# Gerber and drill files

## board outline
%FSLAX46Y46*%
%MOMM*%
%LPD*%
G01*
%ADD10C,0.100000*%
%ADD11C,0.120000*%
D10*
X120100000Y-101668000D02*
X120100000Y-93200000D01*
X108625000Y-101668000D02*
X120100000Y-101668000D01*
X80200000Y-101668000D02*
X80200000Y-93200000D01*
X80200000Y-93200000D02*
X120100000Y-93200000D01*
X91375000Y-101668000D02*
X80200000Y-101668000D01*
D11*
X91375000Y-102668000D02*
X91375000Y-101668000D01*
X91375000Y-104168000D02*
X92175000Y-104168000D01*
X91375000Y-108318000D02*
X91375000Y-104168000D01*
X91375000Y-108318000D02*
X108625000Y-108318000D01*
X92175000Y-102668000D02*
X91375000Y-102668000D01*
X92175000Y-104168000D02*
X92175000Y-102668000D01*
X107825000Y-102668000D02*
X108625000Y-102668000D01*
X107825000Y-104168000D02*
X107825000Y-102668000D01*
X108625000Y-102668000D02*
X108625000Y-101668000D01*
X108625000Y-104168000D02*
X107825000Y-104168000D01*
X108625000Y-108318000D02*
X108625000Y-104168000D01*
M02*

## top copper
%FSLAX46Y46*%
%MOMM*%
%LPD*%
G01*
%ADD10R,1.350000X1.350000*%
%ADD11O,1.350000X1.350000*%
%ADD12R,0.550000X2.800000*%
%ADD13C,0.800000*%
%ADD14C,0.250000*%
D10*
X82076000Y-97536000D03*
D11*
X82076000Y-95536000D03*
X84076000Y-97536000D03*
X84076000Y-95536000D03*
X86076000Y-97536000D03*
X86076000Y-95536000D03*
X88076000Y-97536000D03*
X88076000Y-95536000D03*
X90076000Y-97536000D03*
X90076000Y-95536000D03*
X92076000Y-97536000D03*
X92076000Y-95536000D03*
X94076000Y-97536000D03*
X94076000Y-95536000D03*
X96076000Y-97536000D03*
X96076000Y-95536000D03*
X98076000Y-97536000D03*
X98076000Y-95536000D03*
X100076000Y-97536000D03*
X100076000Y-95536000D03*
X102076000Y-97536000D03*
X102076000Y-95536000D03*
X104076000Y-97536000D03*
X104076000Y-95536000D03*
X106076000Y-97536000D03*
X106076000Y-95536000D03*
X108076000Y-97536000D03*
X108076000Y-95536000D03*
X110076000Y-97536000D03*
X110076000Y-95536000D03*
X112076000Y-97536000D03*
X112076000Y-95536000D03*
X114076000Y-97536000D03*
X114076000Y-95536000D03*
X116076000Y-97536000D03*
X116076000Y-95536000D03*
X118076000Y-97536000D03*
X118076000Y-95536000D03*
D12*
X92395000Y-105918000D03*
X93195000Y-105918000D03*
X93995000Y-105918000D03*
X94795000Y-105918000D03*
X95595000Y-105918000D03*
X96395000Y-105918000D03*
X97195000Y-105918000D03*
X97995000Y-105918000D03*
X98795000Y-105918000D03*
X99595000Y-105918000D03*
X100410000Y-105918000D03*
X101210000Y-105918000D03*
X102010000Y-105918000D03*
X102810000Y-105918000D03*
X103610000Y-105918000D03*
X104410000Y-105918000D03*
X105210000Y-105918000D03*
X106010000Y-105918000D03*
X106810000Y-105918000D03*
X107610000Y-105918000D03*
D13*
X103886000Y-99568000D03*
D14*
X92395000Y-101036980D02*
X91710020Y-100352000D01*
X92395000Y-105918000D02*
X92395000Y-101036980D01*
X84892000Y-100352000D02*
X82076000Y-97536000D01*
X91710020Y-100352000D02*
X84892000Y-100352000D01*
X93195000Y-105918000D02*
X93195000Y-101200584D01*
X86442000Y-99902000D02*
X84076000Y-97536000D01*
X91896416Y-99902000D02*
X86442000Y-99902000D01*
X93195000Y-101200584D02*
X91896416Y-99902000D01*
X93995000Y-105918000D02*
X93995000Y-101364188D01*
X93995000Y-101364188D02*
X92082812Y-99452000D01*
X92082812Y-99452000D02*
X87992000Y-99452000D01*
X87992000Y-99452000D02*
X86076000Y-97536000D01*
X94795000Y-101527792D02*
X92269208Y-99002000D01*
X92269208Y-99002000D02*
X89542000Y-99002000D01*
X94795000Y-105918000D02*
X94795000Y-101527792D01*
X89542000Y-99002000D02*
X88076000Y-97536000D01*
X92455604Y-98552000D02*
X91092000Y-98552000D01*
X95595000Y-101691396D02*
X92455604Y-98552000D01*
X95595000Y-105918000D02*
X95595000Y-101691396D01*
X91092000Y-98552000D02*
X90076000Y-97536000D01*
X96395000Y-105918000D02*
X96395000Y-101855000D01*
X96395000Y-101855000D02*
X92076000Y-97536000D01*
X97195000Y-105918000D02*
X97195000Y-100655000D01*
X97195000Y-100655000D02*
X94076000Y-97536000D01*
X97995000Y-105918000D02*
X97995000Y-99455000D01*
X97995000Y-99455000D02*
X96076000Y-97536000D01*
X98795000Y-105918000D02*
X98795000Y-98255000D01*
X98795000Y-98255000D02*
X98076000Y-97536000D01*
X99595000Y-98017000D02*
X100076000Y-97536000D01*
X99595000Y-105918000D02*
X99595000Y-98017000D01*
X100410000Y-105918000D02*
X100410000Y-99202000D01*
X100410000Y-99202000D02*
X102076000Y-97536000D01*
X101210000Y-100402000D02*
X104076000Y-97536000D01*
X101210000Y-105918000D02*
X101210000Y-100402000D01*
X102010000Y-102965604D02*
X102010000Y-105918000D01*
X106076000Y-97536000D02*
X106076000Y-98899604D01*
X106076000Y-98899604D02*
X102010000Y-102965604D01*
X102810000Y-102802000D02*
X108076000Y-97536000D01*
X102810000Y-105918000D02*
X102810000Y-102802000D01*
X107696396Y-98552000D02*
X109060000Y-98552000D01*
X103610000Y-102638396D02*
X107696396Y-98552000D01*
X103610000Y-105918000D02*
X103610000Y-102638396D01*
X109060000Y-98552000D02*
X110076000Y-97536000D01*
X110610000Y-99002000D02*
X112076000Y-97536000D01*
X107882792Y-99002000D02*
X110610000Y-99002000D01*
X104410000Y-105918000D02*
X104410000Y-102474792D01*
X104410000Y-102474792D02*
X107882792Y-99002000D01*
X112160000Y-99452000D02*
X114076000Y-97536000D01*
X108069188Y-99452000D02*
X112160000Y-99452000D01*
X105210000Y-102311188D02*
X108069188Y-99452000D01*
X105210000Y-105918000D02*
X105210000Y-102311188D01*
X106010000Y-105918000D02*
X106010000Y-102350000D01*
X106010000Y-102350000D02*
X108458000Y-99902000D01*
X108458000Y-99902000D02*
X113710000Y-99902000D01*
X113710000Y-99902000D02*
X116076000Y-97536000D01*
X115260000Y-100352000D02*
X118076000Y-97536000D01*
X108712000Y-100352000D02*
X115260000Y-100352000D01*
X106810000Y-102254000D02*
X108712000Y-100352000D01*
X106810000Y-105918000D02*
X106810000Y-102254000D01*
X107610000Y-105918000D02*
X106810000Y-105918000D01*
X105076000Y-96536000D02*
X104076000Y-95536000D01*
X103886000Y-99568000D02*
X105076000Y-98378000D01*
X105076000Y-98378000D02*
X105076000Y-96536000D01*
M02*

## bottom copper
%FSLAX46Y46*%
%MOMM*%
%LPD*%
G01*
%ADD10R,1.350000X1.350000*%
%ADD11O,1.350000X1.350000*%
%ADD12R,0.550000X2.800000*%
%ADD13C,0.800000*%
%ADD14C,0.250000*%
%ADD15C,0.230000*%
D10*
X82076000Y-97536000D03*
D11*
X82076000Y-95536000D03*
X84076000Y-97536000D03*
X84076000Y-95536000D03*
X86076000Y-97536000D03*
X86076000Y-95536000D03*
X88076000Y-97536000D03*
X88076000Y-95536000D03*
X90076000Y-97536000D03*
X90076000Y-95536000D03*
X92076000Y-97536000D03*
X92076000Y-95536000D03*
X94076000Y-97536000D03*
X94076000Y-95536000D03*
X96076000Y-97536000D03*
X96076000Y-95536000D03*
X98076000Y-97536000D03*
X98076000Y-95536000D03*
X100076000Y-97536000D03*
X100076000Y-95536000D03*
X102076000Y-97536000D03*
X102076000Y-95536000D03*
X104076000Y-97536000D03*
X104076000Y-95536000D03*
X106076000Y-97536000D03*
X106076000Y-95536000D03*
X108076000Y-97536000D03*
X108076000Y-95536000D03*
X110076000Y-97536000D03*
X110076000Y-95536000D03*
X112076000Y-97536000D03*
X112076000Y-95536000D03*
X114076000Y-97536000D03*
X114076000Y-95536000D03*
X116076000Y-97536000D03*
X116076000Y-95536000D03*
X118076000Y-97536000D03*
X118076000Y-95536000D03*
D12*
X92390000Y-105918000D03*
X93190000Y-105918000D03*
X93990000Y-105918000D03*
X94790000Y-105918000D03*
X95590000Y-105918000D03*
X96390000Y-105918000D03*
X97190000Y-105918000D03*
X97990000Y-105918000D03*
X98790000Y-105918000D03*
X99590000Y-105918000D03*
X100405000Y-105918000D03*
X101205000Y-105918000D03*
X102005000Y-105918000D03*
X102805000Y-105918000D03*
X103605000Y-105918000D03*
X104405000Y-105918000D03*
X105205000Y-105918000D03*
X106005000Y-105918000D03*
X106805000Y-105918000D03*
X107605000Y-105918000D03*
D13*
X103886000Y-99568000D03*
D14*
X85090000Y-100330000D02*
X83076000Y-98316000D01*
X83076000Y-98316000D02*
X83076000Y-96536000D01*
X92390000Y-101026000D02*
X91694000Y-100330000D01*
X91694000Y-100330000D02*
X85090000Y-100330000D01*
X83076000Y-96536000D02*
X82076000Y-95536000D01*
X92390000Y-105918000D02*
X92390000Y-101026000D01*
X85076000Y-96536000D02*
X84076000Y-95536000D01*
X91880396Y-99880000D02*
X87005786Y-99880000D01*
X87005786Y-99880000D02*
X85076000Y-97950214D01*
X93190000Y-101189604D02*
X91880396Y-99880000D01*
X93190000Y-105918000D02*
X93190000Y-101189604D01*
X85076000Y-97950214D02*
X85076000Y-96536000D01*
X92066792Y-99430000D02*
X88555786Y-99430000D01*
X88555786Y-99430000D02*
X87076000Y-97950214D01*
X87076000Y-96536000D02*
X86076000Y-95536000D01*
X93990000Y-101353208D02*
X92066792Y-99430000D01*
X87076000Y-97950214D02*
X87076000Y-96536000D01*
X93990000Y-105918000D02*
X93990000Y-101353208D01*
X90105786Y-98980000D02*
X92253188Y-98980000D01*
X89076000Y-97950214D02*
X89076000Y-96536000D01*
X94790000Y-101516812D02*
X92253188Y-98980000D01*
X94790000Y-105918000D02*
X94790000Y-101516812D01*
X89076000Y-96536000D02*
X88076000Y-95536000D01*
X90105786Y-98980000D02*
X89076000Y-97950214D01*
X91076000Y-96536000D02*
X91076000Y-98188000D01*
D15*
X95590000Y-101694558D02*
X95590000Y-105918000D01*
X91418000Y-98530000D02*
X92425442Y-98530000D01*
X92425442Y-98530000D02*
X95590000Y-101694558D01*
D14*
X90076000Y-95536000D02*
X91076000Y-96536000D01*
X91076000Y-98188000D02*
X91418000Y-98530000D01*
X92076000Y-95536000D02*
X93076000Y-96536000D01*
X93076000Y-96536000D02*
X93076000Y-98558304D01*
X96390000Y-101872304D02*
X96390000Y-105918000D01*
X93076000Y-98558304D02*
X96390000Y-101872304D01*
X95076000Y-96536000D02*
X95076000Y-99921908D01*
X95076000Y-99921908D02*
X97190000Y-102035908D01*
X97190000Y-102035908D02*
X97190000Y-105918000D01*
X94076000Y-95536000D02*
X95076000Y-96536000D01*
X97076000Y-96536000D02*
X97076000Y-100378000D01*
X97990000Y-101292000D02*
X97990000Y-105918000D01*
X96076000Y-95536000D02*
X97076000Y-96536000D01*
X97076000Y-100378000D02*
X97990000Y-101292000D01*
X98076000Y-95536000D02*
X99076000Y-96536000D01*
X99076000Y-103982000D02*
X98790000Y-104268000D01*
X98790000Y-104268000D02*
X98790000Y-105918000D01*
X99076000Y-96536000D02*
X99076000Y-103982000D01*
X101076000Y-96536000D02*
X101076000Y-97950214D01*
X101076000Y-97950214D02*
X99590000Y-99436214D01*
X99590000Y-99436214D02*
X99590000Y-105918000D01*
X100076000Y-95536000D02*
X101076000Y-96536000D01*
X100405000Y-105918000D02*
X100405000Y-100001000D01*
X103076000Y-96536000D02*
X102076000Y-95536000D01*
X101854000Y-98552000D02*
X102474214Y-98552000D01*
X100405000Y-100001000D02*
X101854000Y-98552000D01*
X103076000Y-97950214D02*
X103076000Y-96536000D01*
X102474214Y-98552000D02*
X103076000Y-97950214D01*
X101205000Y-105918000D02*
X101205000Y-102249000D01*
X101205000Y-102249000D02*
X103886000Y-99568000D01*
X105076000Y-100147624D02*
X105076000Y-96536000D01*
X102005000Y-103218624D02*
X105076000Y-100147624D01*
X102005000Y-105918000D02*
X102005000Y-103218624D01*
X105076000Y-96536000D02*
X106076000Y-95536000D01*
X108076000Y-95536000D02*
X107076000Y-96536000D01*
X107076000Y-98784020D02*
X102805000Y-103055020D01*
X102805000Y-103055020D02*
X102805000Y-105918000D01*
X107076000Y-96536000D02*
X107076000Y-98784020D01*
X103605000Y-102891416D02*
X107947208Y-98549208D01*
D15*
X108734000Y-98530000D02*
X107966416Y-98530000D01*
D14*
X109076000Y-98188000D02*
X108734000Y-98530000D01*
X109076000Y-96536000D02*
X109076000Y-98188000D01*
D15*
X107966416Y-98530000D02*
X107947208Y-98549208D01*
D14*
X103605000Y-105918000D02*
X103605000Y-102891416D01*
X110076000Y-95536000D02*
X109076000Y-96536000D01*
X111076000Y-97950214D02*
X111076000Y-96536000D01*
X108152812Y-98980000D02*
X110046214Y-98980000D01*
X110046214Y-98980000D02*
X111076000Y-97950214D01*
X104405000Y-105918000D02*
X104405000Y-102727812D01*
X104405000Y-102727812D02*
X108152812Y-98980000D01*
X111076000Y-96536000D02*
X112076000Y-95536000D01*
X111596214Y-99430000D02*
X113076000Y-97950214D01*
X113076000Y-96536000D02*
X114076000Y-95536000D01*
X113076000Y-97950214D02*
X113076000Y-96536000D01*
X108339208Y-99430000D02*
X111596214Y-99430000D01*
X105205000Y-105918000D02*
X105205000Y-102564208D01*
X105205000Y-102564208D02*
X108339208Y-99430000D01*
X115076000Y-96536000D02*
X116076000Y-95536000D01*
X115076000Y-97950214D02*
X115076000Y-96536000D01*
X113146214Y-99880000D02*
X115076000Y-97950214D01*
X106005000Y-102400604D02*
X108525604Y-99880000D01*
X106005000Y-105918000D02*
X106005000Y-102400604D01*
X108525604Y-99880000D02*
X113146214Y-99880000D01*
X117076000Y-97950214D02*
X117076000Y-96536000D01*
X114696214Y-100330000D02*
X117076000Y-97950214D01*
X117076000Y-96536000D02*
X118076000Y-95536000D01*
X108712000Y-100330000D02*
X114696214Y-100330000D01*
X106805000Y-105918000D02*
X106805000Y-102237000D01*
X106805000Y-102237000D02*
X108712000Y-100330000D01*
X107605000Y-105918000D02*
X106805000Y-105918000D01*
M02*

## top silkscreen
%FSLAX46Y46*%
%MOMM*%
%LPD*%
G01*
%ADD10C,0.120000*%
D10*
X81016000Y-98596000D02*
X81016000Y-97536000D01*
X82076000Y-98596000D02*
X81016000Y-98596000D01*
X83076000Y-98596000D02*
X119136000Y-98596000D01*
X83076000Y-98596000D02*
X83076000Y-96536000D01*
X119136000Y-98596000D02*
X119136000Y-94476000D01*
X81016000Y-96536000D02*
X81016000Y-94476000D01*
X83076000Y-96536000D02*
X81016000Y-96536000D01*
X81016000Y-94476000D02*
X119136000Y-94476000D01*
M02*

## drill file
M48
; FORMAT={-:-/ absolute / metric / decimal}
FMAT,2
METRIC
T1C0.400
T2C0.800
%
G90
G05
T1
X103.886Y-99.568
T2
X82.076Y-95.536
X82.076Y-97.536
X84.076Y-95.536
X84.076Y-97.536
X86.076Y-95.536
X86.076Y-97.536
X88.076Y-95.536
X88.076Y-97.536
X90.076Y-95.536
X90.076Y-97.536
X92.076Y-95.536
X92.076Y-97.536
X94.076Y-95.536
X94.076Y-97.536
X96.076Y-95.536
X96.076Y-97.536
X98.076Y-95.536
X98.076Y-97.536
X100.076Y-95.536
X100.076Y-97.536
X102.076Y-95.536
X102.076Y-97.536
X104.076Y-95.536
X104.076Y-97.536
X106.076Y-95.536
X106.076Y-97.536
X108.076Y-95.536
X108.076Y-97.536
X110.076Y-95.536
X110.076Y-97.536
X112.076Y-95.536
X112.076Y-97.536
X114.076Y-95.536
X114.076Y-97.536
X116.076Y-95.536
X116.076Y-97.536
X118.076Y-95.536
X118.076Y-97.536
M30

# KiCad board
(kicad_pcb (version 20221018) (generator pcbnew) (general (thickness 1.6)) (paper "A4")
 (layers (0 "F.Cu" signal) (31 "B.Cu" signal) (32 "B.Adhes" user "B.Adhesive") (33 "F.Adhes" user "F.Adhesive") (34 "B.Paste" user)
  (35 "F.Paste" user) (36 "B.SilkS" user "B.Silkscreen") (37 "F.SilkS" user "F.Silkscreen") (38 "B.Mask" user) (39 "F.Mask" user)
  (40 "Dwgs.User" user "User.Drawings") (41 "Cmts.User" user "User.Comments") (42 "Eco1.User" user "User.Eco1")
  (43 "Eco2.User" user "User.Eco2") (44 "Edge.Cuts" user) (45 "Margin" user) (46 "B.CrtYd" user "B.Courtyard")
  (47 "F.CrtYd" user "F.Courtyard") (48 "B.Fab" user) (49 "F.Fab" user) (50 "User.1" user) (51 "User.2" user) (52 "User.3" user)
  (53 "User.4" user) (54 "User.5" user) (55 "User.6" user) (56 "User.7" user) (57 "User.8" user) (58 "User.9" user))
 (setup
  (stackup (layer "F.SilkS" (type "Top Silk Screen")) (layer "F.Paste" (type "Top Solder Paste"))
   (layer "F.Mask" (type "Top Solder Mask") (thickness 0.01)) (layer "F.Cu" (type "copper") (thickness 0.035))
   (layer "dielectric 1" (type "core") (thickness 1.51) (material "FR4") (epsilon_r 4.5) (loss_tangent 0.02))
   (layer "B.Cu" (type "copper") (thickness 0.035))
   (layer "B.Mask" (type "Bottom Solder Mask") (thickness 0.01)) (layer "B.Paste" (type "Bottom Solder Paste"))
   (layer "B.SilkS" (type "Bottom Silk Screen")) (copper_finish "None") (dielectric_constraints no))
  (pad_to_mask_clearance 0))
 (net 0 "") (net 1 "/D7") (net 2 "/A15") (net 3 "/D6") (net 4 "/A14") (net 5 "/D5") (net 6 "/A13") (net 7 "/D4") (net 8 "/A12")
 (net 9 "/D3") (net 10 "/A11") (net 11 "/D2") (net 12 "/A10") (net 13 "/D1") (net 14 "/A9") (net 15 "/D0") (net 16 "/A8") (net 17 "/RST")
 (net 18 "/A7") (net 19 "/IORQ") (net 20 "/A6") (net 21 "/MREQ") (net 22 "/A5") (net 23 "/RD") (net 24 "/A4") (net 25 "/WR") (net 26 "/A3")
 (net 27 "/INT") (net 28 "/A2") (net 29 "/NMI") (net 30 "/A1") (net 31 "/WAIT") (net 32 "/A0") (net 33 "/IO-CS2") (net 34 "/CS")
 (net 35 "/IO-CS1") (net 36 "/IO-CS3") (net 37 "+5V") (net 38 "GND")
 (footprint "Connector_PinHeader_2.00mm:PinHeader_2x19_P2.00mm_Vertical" (layer "F.Cu") (at 82.076 97.536 90)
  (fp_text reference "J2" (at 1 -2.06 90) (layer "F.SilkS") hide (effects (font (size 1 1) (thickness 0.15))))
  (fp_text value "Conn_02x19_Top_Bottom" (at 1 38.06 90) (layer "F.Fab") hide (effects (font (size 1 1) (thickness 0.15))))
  (fp_line (start -1.06 -1.06) (end 0 -1.06) (stroke (width 0.12) (type solid)) (layer "F.SilkS"))
  (fp_line (start -1.06 0) (end -1.06 -1.06) (stroke (width 0.12) (type solid)) (layer "F.SilkS"))
  (fp_line (start -1.06 1) (end -1.06 37.06) (stroke (width 0.12) (type solid)) (layer "F.SilkS"))
  (fp_line (start -1.06 1) (end 1 1) (stroke (width 0.12) (type solid)) (layer "F.SilkS"))
  (fp_line (start -1.06 37.06) (end 3.06 37.06) (stroke (width 0.12) (type solid)) (layer "F.SilkS"))
  (fp_line (start 1 -1.06) (end 3.06 -1.06) (stroke (width 0.12) (type solid)) (layer "F.SilkS"))
  (fp_line (start 1 1) (end 1 -1.06) (stroke (width 0.12) (type solid)) (layer "F.SilkS"))
  (fp_line (start 3.06 -1.06) (end 3.06 37.06) (stroke (width 0.12) (type solid)) (layer "F.SilkS"))
  (pad "1" thru_hole rect (at 0 0 90) (size 1.35 1.35) (drill 0.8) (layers "*.Cu" "*.Mask") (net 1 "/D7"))
  (pad "2" thru_hole oval (at 2 0 90) (size 1.35 1.35) (drill 0.8) (layers "*.Cu" "*.Mask") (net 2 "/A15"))
  (pad "3" thru_hole oval (at 0 2 90) (size 1.35 1.35) (drill 0.8) (layers "*.Cu" "*.Mask") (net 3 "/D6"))
  (pad "4" thru_hole oval (at 2 2 90) (size 1.35 1.35) (drill 0.8) (layers "*.Cu" "*.Mask") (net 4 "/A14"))
  (pad "5" thru_hole oval (at 0 4 90) (size 1.35 1.35) (drill 0.8) (layers "*.Cu" "*.Mask") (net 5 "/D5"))
  (pad "6" thru_hole oval (at 2 4 90) (size 1.35 1.35) (drill 0.8) (layers "*.Cu" "*.Mask") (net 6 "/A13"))
  (pad "7" thru_hole oval (at 0 6 90) (size 1.35 1.35) (drill 0.8) (layers "*.Cu" "*.Mask") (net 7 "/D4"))
  (pad "8" thru_hole oval (at 2 6 90) (size 1.35 1.35) (drill 0.8) (layers "*.Cu" "*.Mask") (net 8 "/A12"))
  (pad "9" thru_hole oval (at 0 8 90) (size 1.35 1.35) (drill 0.8) (layers "*.Cu" "*.Mask") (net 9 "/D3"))
  (pad "10" thru_hole oval (at 2 8 90) (size 1.35 1.35) (drill 0.8) (layers "*.Cu" "*.Mask") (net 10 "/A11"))
  (pad "11" thru_hole oval (at 0 10 90) (size 1.35 1.35) (drill 0.8) (layers "*.Cu" "*.Mask") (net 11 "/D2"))
  (pad "12" thru_hole oval (at 2 10 90) (size 1.35 1.35) (drill 0.8) (layers "*.Cu" "*.Mask") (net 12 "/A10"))
  (pad "13" thru_hole oval (at 0 12 90) (size 1.35 1.35) (drill 0.8) (layers "*.Cu" "*.Mask") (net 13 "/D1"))
  (pad "14" thru_hole oval (at 2 12 90) (size 1.35 1.35) (drill 0.8) (layers "*.Cu" "*.Mask") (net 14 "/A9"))
  (pad "15" thru_hole oval (at 0 14 90) (size 1.35 1.35) (drill 0.8) (layers "*.Cu" "*.Mask") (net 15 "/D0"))
  (pad "16" thru_hole oval (at 2 14 90) (size 1.35 1.35) (drill 0.8) (layers "*.Cu" "*.Mask") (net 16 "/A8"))
  (pad "17" thru_hole oval (at 0 16 90) (size 1.35 1.35) (drill 0.8) (layers "*.Cu" "*.Mask") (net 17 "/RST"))
  (pad "18" thru_hole oval (at 2 16 90) (size 1.35 1.35) (drill 0.8) (layers "*.Cu" "*.Mask") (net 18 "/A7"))
  (pad "19" thru_hole oval (at 0 18 90) (size 1.35 1.35) (drill 0.8) (layers "*.Cu" "*.Mask") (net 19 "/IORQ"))
  (pad "20" thru_hole oval (at 2 18 90) (size 1.35 1.35) (drill 0.8) (layers "*.Cu" "*.Mask") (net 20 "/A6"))
  (pad "21" thru_hole oval (at 0 20 90) (size 1.35 1.35) (drill 0.8) (layers "*.Cu" "*.Mask") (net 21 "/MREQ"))
  (pad "22" thru_hole oval (at 2 20 90) (size 1.35 1.35) (drill 0.8) (layers "*.Cu" "*.Mask") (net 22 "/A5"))
  (pad "23" thru_hole oval (at 0 22 90) (size 1.35 1.35) (drill 0.8) (layers "*.Cu" "*.Mask") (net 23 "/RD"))
  (pad "24" thru_hole oval (at 2 22 90) (size 1.35 1.35) (drill 0.8) (layers "*.Cu" "*.Mask") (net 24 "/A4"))
  (pad "25" thru_hole oval (at 0 24 90) (size 1.35 1.35) (drill 0.8) (layers "*.Cu" "*.Mask") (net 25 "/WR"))
  (pad "26" thru_hole oval (at 2 24 90) (size 1.35 1.35) (drill 0.8) (layers "*.Cu" "*.Mask") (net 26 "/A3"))
  (pad "27" thru_hole oval (at 0 26 90) (size 1.35 1.35) (drill 0.8) (layers "*.Cu" "*.Mask") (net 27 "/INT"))
  (pad "28" thru_hole oval (at 2 26 90) (size 1.35 1.35) (drill 0.8) (layers "*.Cu" "*.Mask") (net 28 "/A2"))
  (pad "29" thru_hole oval (at 0 28 90) (size 1.35 1.35) (drill 0.8) (layers "*.Cu" "*.Mask") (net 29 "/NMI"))
  (pad "30" thru_hole oval (at 2 28 90) (size 1.35 1.35) (drill 0.8) (layers "*.Cu" "*.Mask") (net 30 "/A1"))
  (pad "31" thru_hole oval (at 0 30 90) (size 1.35 1.35) (drill 0.8) (layers "*.Cu" "*.Mask") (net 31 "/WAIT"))
  (pad "32" thru_hole oval (at 2 30 90) (size 1.35 1.35) (drill 0.8) (layers "*.Cu" "*.Mask") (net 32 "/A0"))
  (pad "33" thru_hole oval (at 0 32 90) (size 1.35 1.35) (drill 0.8) (layers "*.Cu" "*.Mask") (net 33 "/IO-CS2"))
  (pad "34" thru_hole oval (at 2 32 90) (size 1.35 1.35) (drill 0.8) (layers "*.Cu" "*.Mask") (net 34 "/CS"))
  (pad "35" thru_hole oval (at 0 34 90) (size 1.35 1.35) (drill 0.8) (layers "*.Cu" "*.Mask") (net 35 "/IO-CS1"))
  (pad "36" thru_hole oval (at 2 34 90) (size 1.35 1.35) (drill 0.8) (layers "*.Cu" "*.Mask") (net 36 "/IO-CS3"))
  (pad "37" thru_hole oval (at 0 36 90) (size 1.35 1.35) (drill 0.8) (layers "*.Cu" "*.Mask") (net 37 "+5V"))
  (pad "38" thru_hole oval (at 2 36 90) (size 1.35 1.35) (drill 0.8) (layers "*.Cu" "*.Mask") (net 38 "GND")))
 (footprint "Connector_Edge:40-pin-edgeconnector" (layer "F.Cu") (at 100 103.378)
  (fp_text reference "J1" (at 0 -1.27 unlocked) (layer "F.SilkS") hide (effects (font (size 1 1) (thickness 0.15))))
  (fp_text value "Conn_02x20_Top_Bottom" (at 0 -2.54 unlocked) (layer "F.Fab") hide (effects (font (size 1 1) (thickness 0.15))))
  (fp_line (start -8.625 -0.71) (end -8.625 -1.71) (stroke (width 0.12) (type default)) (layer "Edge.Cuts"))
  (fp_line (start -8.625 0.79) (end -7.825 0.79) (stroke (width 0.12) (type default)) (layer "Edge.Cuts"))
  (fp_line (start -8.625 4.94) (end -8.625 0.79) (stroke (width 0.12) (type default)) (layer "Edge.Cuts"))
  (fp_line (start -8.625 4.94) (end 8.625 4.94) (stroke (width 0.12) (type default)) (layer "Edge.Cuts"))
  (fp_line (start -7.825 -0.71) (end -8.625 -0.71) (stroke (width 0.12) (type default)) (layer "Edge.Cuts"))
  (fp_line (start -7.825 0.79) (end -7.825 -0.71) (stroke (width 0.12) (type default)) (layer "Edge.Cuts"))
  (fp_line (start 7.825 -0.71) (end 8.625 -0.71) (stroke (width 0.12) (type default)) (layer "Edge.Cuts"))
  (fp_line (start 7.825 0.79) (end 7.825 -0.71) (stroke (width 0.12) (type default)) (layer "Edge.Cuts"))
  (fp_line (start 8.625 -0.71) (end 8.625 -1.71) (stroke (width 0.12) (type default)) (layer "Edge.Cuts"))
  (fp_line (start 8.625 0.79) (end 7.825 0.79) (stroke (width 0.12) (type default)) (layer "Edge.Cuts"))
  (fp_line (start 8.625 4.94) (end 8.625 0.79) (stroke (width 0.12) (type default)) (layer "Edge.Cuts"))
  (pad "1" smd rect (at -7.605 2.54 90) (size 2.8 0.55) (layers "F.Cu" "F.Paste" "F.Mask") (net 1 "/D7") (thermal_bridge_angle 45))
  (pad "2" smd rect (at -6.805 2.54 90) (size 2.8 0.55) (layers "F.Cu" "F.Paste" "F.Mask") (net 3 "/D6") (thermal_bridge_angle 45))
  (pad "3" smd rect (at -6.005 2.54 90) (size 2.8 0.55) (layers "F.Cu" "F.Paste" "F.Mask") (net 5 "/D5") (thermal_bridge_angle 45))
  (pad "4" smd rect (at -5.205 2.54 90) (size 2.8 0.55) (layers "F.Cu" "F.Paste" "F.Mask") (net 7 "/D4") (thermal_bridge_angle 45))
  (pad "5" smd rect (at -4.405 2.54 90) (size 2.8 0.55) (layers "F.Cu" "F.Paste" "F.Mask") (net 9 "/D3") (thermal_bridge_angle 45))
  (pad "6" smd rect (at -3.605 2.54 90) (size 2.8 0.55) (layers "F.Cu" "F.Paste" "F.Mask") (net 11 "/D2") (thermal_bridge_angle 45))
  (pad "7" smd rect (at -2.805 2.54 90) (size 2.8 0.55) (layers "F.Cu" "F.Paste" "F.Mask") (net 13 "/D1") (thermal_bridge_angle 45))
  (pad "8" smd rect (at -2.005 2.54 90) (size 2.8 0.55) (layers "F.Cu" "F.Paste" "F.Mask") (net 15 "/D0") (thermal_bridge_angle 45))
  (pad "9" smd rect (at -1.205 2.54 90) (size 2.8 0.55) (layers "F.Cu" "F.Paste" "F.Mask") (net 17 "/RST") (thermal_bridge_angle 45))
  (pad "10" smd rect (at -0.405 2.54 90) (size 2.8 0.55) (layers "F.Cu" "F.Paste" "F.Mask") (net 19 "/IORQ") (thermal_bridge_angle 45))
  (pad "11" smd rect (at 0.41 2.54 90) (size 2.8 0.55) (layers "F.Cu" "F.Paste" "F.Mask") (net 21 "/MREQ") (thermal_bridge_angle 45))
  (pad "12" smd rect (at 1.21 2.54 90) (size 2.8 0.55) (layers "F.Cu" "F.Paste" "F.Mask") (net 23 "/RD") (thermal_bridge_angle 45))
  (pad "13" smd rect (at 2.01 2.54 90) (size 2.8 0.55) (layers "F.Cu" "F.Paste" "F.Mask") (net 25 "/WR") (thermal_bridge_angle 45))
  (pad "14" smd rect (at 2.81 2.54 90) (size 2.8 0.55) (layers "F.Cu" "F.Paste" "F.Mask") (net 27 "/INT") (thermal_bridge_angle 45))
  (pad "15" smd rect (at 3.61 2.54 90) (size 2.8 0.55) (layers "F.Cu" "F.Paste" "F.Mask") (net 29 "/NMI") (thermal_bridge_angle 45))
  (pad "16" smd rect (at 4.41 2.54 90) (size 2.8 0.55) (layers "F.Cu" "F.Paste" "F.Mask") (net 31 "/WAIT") (thermal_bridge_angle 45))
  (pad "17" smd rect (at 5.21 2.54 90) (size 2.8 0.55) (layers "F.Cu" "F.Paste" "F.Mask") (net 33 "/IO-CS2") (thermal_bridge_angle 45))
  (pad "18" smd rect (at 6.01 2.54 90) (size 2.8 0.55) (layers "F.Cu" "F.Paste" "F.Mask") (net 35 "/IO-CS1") (thermal_bridge_angle 45))
  (pad "19" smd rect (at 6.81 2.54 90) (size 2.8 0.55) (layers "F.Cu" "F.Paste" "F.Mask") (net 37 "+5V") (thermal_bridge_angle 45))
  (pad "20" smd rect (at 7.61 2.54 90) (size 2.8 0.55) (layers "F.Cu" "F.Paste" "F.Mask") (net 37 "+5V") (thermal_bridge_angle 45))
  (pad "21" smd rect (at -7.61 2.54 270) (size 2.8 0.55) (layers "B.Cu" "B.Paste" "B.Mask") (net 2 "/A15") (thermal_bridge_angle 45))
  (pad "22" smd rect (at -6.81 2.54 270) (size 2.8 0.55) (layers "B.Cu" "B.Paste" "B.Mask") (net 4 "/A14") (thermal_bridge_angle 45))
  (pad "23" smd rect (at -6.01 2.54 270) (size 2.8 0.55) (layers "B.Cu" "B.Paste" "B.Mask") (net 6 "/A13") (thermal_bridge_angle 45))
  (pad "24" smd rect (at -5.21 2.54 270) (size 2.8 0.55) (layers "B.Cu" "B.Paste" "B.Mask") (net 8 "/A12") (thermal_bridge_angle 45))
  (pad "25" smd rect (at -4.41 2.54 270) (size 2.8 0.55) (layers "B.Cu" "B.Paste" "B.Mask") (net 10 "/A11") (thermal_bridge_angle 45))
  (pad "26" smd rect (at -3.61 2.54 270) (size 2.8 0.55) (layers "B.Cu" "B.Paste" "B.Mask") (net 12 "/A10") (thermal_bridge_angle 45))
  (pad "27" smd rect (at -2.81 2.54 270) (size 2.8 0.55) (layers "B.Cu" "B.Paste" "B.Mask") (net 14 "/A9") (thermal_bridge_angle 45))
  (pad "28" smd rect (at -2.01 2.54 270) (size 2.8 0.55) (layers "B.Cu" "B.Paste" "B.Mask") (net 16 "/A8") (thermal_bridge_angle 45))
  (pad "29" smd rect (at -1.21 2.54 270) (size 2.8 0.55) (layers "B.Cu" "B.Paste" "B.Mask") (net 18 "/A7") (thermal_bridge_angle 45))
  (pad "30" smd rect (at -0.41 2.54 270) (size 2.8 0.55) (layers "B.Cu" "B.Paste" "B.Mask") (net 20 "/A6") (thermal_bridge_angle 45))
  (pad "31" smd rect (at 0.405 2.54 270) (size 2.8 0.55) (layers "B.Cu" "B.Paste" "B.Mask") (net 22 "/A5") (thermal_bridge_angle 45))
  (pad "32" smd rect (at 1.205 2.54 270) (size 2.8 0.55) (layers "B.Cu" "B.Paste" "B.Mask") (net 24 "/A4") (thermal_bridge_angle 45))
  (pad "33" smd rect (at 2.005 2.54 270) (size 2.8 0.55) (layers "B.Cu" "B.Paste" "B.Mask") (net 26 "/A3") (thermal_bridge_angle 45))
  (pad "34" smd rect (at 2.805 2.54 270) (size 2.8 0.55) (layers "B.Cu" "B.Paste" "B.Mask") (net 28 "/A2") (thermal_bridge_angle 45))
  (pad "35" smd rect (at 3.605 2.54 270) (size 2.8 0.55) (layers "B.Cu" "B.Paste" "B.Mask") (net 30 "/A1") (thermal_bridge_angle 45))
  (pad "36" smd rect (at 4.405 2.54 270) (size 2.8 0.55) (layers "B.Cu" "B.Paste" "B.Mask") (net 32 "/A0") (thermal_bridge_angle 45))
  (pad "37" smd rect (at 5.205 2.54 270) (size 2.8 0.55) (layers "B.Cu" "B.Paste" "B.Mask") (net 34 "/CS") (thermal_bridge_angle 45))
  (pad "38" smd rect (at 6.005 2.54 270) (size 2.8 0.55) (layers "B.Cu" "B.Paste" "B.Mask") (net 36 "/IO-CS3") (thermal_bridge_angle 45))
  (pad "39" smd rect (at 6.805 2.54 270) (size 2.8 0.55) (layers "B.Cu" "B.Paste" "B.Mask") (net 38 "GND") (thermal_bridge_angle 45))
  (pad "40" smd rect (at 7.605 2.54 270) (size 2.8 0.55) (layers "B.Cu" "B.Paste" "B.Mask") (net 38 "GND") (thermal_bridge_angle 45)))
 (gr_line (start 120.1 101.668) (end 120.1 93.2) (stroke (width 0.1) (type default)) (layer "Edge.Cuts"))
 (gr_line (start 108.625 101.668) (end 120.1 101.668) (stroke (width 0.1) (type default)) (layer "Edge.Cuts"))
 (gr_line (start 80.2 101.668) (end 80.2 93.2) (stroke (width 0.1) (type default)) (layer "Edge.Cuts"))
 (gr_line (start 80.2 93.2) (end 120.1 93.2) (stroke (width 0.1) (type default)) (layer "Edge.Cuts"))
 (gr_line (start 91.375 101.668) (end 80.2 101.668) (stroke (width 0.1) (type default)) (layer "Edge.Cuts"))
 (segment (start 92.395 101.03698) (end 91.71002 100.352) (width 0.25) (layer "F.Cu") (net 1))
 (segment (start 92.395 105.918) (end 92.395 101.03698) (width 0.25) (layer "F.Cu") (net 1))
 (segment (start 84.892 100.352) (end 82.076 97.536) (width 0.25) (layer "F.Cu") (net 1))
 (segment (start 91.71002 100.352) (end 84.892 100.352) (width 0.25) (layer "F.Cu") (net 1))
 (segment (start 93.195 105.918) (end 93.195 101.200584) (width 0.25) (layer "F.Cu") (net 3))
 (segment (start 86.442 99.902) (end 84.076 97.536) (width 0.25) (layer "F.Cu") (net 3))
 (segment (start 91.896416 99.902) (end 86.442 99.902) (width 0.25) (layer "F.Cu") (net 3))
 (segment (start 93.195 101.200584) (end 91.896416 99.902) (width 0.25) (layer "F.Cu") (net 3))
 (segment (start 93.995 105.918) (end 93.995 101.364188) (width 0.25) (layer "F.Cu") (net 5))
 (segment (start 93.995 101.364188) (end 92.082812 99.452) (width 0.25) (layer "F.Cu") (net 5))
 (segment (start 92.082812 99.452) (end 87.992 99.452) (width 0.25) (layer "F.Cu") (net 5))
 (segment (start 87.992 99.452) (end 86.076 97.536) (width 0.25) (layer "F.Cu") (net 5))
 (segment (start 94.795 101.527792) (end 92.269208 99.002) (width 0.25) (layer "F.Cu") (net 7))
 (segment (start 92.269208 99.002) (end 89.542 99.002) (width 0.25) (layer "F.Cu") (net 7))
 (segment (start 94.795 105.918) (end 94.795 101.527792) (width 0.25) (layer "F.Cu") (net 7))
 (segment (start 89.542 99.002) (end 88.076 97.536) (width 0.25) (layer "F.Cu") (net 7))
 (segment (start 92.455604 98.552) (end 91.092 98.552) (width 0.25) (layer "F.Cu") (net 9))
 (segment (start 95.595 101.691396) (end 92.455604 98.552) (width 0.25) (layer "F.Cu") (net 9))
 (segment (start 95.595 105.918) (end 95.595 101.691396) (width 0.25) (layer "F.Cu") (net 9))
 (segment (start 91.092 98.552) (end 90.076 97.536) (width 0.25) (layer "F.Cu") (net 9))
 (segment (start 96.395 105.918) (end 96.395 101.855) (width 0.25) (layer "F.Cu") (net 11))
 (segment (start 96.395 101.855) (end 92.076 97.536) (width 0.25) (layer "F.Cu") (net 11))
 (segment (start 97.195 105.918) (end 97.195 100.655) (width 0.25) (layer "F.Cu") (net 13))
 (segment (start 97.195 100.655) (end 94.076 97.536) (width 0.25) (layer "F.Cu") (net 13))
 (segment (start 97.995 105.918) (end 97.995 99.455) (width 0.25) (layer "F.Cu") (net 15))
 (segment (start 97.995 99.455) (end 96.076 97.536) (width 0.25) (layer "F.Cu") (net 15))
 (segment (start 98.795 105.918) (end 98.795 98.255) (width 0.25) (layer "F.Cu") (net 17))
 (segment (start 98.795 98.255) (end 98.076 97.536) (width 0.25) (layer "F.Cu") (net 17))
 (segment (start 99.595 98.017) (end 100.076 97.536) (width 0.25) (layer "F.Cu") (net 19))
 (segment (start 99.595 105.918) (end 99.595 98.017) (width 0.25) (layer "F.Cu") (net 19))
 (segment (start 100.41 105.918) (end 100.41 99.202) (width 0.25) (layer "F.Cu") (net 21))
 (segment (start 100.41 99.202) (end 102.076 97.536) (width 0.25) (layer "F.Cu") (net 21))
 (segment (start 101.21 100.402) (end 104.076 97.536) (width 0.25) (layer "F.Cu") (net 23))
 (segment (start 101.21 105.918) (end 101.21 100.402) (width 0.25) (layer "F.Cu") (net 23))
 (segment (start 102.01 102.965604) (end 102.01 105.918) (width 0.25) (layer "F.Cu") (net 25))
 (segment (start 106.076 97.536) (end 106.076 98.899604) (width 0.25) (layer "F.Cu") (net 25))
 (segment (start 106.076 98.899604) (end 102.01 102.965604) (width 0.25) (layer "F.Cu") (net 25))
 (segment (start 102.81 102.802) (end 108.076 97.536) (width 0.25) (layer "F.Cu") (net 27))
 (segment (start 102.81 105.918) (end 102.81 102.802) (width 0.25) (layer "F.Cu") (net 27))
 (segment (start 107.696396 98.552) (end 109.06 98.552) (width 0.25) (layer "F.Cu") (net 29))
 (segment (start 103.61 102.638396) (end 107.696396 98.552) (width 0.25) (layer "F.Cu") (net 29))
 (segment (start 103.61 105.918) (end 103.61 102.638396) (width 0.25) (layer "F.Cu") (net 29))
 (segment (start 109.06 98.552) (end 110.076 97.536) (width 0.25) (layer "F.Cu") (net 29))
 (segment (start 110.61 99.002) (end 112.076 97.536) (width 0.25) (layer "F.Cu") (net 31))
 (segment (start 107.882792 99.002) (end 110.61 99.002) (width 0.25) (layer "F.Cu") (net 31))
 (segment (start 104.41 105.918) (end 104.41 102.474792) (width 0.25) (layer "F.Cu") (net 31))
 (segment (start 104.41 102.474792) (end 107.882792 99.002) (width 0.25) (layer "F.Cu") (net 31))
 (segment (start 112.16 99.452) (end 114.076 97.536) (width 0.25) (layer "F.Cu") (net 33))
 (segment (start 108.069188 99.452) (end 112.16 99.452) (width 0.25) (layer "F.Cu") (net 33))
 (segment (start 105.21 102.311188) (end 108.069188 99.452) (width 0.25) (layer "F.Cu") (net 33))
 (segment (start 105.21 105.918) (end 105.21 102.311188) (width 0.25) (layer "F.Cu") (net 33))
 (segment (start 106.01 105.918) (end 106.01 102.35) (width 0.25) (layer "F.Cu") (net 35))
 (segment (start 106.01 102.35) (end 108.458 99.902) (width 0.25) (layer "F.Cu") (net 35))
 (segment (start 108.458 99.902) (end 113.71 99.902) (width 0.25) (layer "F.Cu") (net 35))
 (segment (start 113.71 99.902) (end 116.076 97.536) (width 0.25) (layer "F.Cu") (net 35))
 (segment (start 115.26 100.352) (end 118.076 97.536) (width 0.25) (layer "F.Cu") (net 37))
 (segment (start 108.712 100.352) (end 115.26 100.352) (width 0.25) (layer "F.Cu") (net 37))
 (segment (start 106.81 102.254) (end 108.712 100.352) (width 0.25) (layer "F.Cu") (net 37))
 (segment (start 106.81 105.918) (end 106.81 102.254) (width 0.25) (layer "F.Cu") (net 37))
 (segment (start 107.61 105.918) (end 106.81 105.918) (width 0.25) (layer "F.Cu") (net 37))
 (segment (start 85.09 100.33) (end 83.076 98.316) (width 0.25) (layer "B.Cu") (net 2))
 (segment (start 83.076 98.316) (end 83.076 96.536) (width 0.25) (layer "B.Cu") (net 2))
 (segment (start 92.39 101.026) (end 91.694 100.33) (width 0.25) (layer "B.Cu") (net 2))
 (segment (start 91.694 100.33) (end 85.09 100.33) (width 0.25) (layer "B.Cu") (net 2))
 (segment (start 83.076 96.536) (end 82.076 95.536) (width 0.25) (layer "B.Cu") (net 2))
 (segment (start 92.39 105.918) (end 92.39 101.026) (width 0.25) (layer "B.Cu") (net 2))
 (segment (start 85.076 96.536) (end 84.076 95.536) (width 0.25) (layer "B.Cu") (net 4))
 (segment (start 91.880396 99.88) (end 87.005786 99.88) (width 0.25) (layer "B.Cu") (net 4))
 (segment (start 87.005786 99.88) (end 85.076 97.950214) (width 0.25) (layer "B.Cu") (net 4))
 (segment (start 93.19 101.189604) (end 91.880396 99.88) (width 0.25) (layer "B.Cu") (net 4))
 (segment (start 93.19 105.918) (end 93.19 101.189604) (width 0.25) (layer "B.Cu") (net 4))
 (segment (start 85.076 97.950214) (end 85.076 96.536) (width 0.25) (layer "B.Cu") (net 4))
 (segment (start 92.066792 99.43) (end 88.555786 99.43) (width 0.25) (layer "B.Cu") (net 6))
 (segment (start 88.555786 99.43) (end 87.076 97.950214) (width 0.25) (layer "B.Cu") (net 6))
 (segment (start 87.076 96.536) (end 86.076 95.536) (width 0.25) (layer "B.Cu") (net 6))
 (segment (start 93.99 101.353208) (end 92.066792 99.43) (width 0.25) (layer "B.Cu") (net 6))
 (segment (start 87.076 97.950214) (end 87.076 96.536) (width 0.25) (layer "B.Cu") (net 6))
 (segment (start 93.99 105.918) (end 93.99 101.353208) (width 0.25) (layer "B.Cu") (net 6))
 (segment (start 90.105786 98.98) (end 92.253188 98.98) (width 0.25) (layer "B.Cu") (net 8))
 (segment (start 89.076 97.950214) (end 89.076 96.536) (width 0.25) (layer "B.Cu") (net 8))
 (segment (start 94.79 101.516812) (end 92.253188 98.98) (width 0.25) (layer "B.Cu") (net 8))
 (segment (start 94.79 105.918) (end 94.79 101.516812) (width 0.25) (layer "B.Cu") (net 8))
 (segment (start 89.076 96.536) (end 88.076 95.536) (width 0.25) (layer "B.Cu") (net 8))
 (segment (start 90.105786 98.98) (end 89.076 97.950214) (width 0.25) (layer "B.Cu") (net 8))
 (segment (start 91.076 96.536) (end 91.076 98.188) (width 0.25) (layer "B.Cu") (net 10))
 (segment (start 95.59 101.694558) (end 95.59 105.918) (width 0.23) (layer "B.Cu") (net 10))
 (segment (start 91.418 98.53) (end 92.425442 98.53) (width 0.23) (layer "B.Cu") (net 10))
 (segment (start 92.425442 98.53) (end 95.59 101.694558) (width 0.23) (layer "B.Cu") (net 10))
 (segment (start 90.076 95.536) (end 91.076 96.536) (width 0.25) (layer "B.Cu") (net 10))
 (segment (start 91.076 98.188) (end 91.418 98.53) (width 0.25) (layer "B.Cu") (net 10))
 (segment (start 92.076 95.536) (end 93.076 96.536) (width 0.25) (layer "B.Cu") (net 12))
 (segment (start 93.076 96.536) (end 93.076 98.558304) (width 0.25) (layer "B.Cu") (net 12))
 (segment (start 96.39 101.872304) (end 96.39 105.918) (width 0.25) (layer "B.Cu") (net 12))
 (segment (start 93.076 98.558304) (end 96.39 101.872304) (width 0.25) (layer "B.Cu") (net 12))
 (segment (start 95.076 96.536) (end 95.076 99.921908) (width 0.25) (layer "B.Cu") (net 14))
 (segment (start 95.076 99.921908) (end 97.19 102.035908) (width 0.25) (layer "B.Cu") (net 14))
 (segment (start 97.19 102.035908) (end 97.19 105.918) (width 0.25) (layer "B.Cu") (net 14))
 (segment (start 94.076 95.536) (end 95.076 96.536) (width 0.25) (layer "B.Cu") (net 14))
 (segment (start 97.076 96.536) (end 97.076 100.378) (width 0.25) (layer "B.Cu") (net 16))
 (segment (start 97.99 101.292) (end 97.99 105.918) (width 0.25) (layer "B.Cu") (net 16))
 (segment (start 96.076 95.536) (end 97.076 96.536) (width 0.25) (layer "B.Cu") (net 16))
 (segment (start 97.076 100.378) (end 97.99 101.292) (width 0.25) (layer "B.Cu") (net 16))
 (segment (start 98.076 95.536) (end 99.076 96.536) (width 0.25) (layer "B.Cu") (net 18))
 (segment (start 99.076 103.982) (end 98.79 104.268) (width 0.25) (layer "B.Cu") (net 18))
 (segment (start 98.79 104.268) (end 98.79 105.918) (width 0.25) (layer "B.Cu") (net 18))
 (segment (start 99.076 96.536) (end 99.076 103.982) (width 0.25) (layer "B.Cu") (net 18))
 (segment (start 101.076 96.536) (end 101.076 97.950214) (width 0.25) (layer "B.Cu") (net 20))
 (segment (start 101.076 97.950214) (end 99.59 99.436214) (width 0.25) (layer "B.Cu") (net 20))
 (segment (start 99.59 99.436214) (end 99.59 105.918) (width 0.25) (layer "B.Cu") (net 20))
 (segment (start 100.076 95.536) (end 101.076 96.536) (width 0.25) (layer "B.Cu") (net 20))
 (segment (start 100.405 105.918) (end 100.405 100.001) (width 0.25) (layer "B.Cu") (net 22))
 (segment (start 103.076 96.536) (end 102.076 95.536) (width 0.25) (layer "B.Cu") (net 22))
 (segment (start 101.854 98.552) (end 102.474214 98.552) (width 0.25) (layer "B.Cu") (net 22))
 (segment (start 100.405 100.001) (end 101.854 98.552) (width 0.25) (layer "B.Cu") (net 22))
 (segment (start 103.076 97.950214) (end 103.076 96.536) (width 0.25) (layer "B.Cu") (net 22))
 (segment (start 102.474214 98.552) (end 103.076 97.950214) (width 0.25) (layer "B.Cu") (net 22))
 (segment (start 105.076 96.536) (end 104.076 95.536) (width 0.25) (layer "F.Cu") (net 24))
 (segment (start 103.886 99.568) (end 105.076 98.378) (width 0.25) (layer "F.Cu") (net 24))
 (segment (start 105.076 98.378) (end 105.076 96.536) (width 0.25) (layer "F.Cu") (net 24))
 (via (at 103.886 99.568) (size 0.8) (drill 0.4) (layers "F.Cu" "B.Cu") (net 24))
 (segment (start 101.205 105.918) (end 101.205 102.249) (width 0.25) (layer "B.Cu") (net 24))
 (segment (start 101.205 102.249) (end 103.886 99.568) (width 0.25) (layer "B.Cu") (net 24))
 (segment (start 105.076 100.147624) (end 105.076 96.536) (width 0.25) (layer "B.Cu") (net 26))
 (segment (start 102.005 103.218624) (end 105.076 100.147624) (width 0.25) (layer "B.Cu") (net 26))
 (segment (start 102.005 105.918) (end 102.005 103.218624) (width 0.25) (layer "B.Cu") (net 26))
 (segment (start 105.076 96.536) (end 106.076 95.536) (width 0.25) (layer "B.Cu") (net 26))
 (segment (start 108.076 95.536) (end 107.076 96.536) (width 0.25) (layer "B.Cu") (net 28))
 (segment (start 107.076 98.78402) (end 102.805 103.05502) (width 0.25) (layer "B.Cu") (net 28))
 (segment (start 102.805 103.05502) (end 102.805 105.918) (width 0.25) (layer "B.Cu") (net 28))
 (segment (start 107.076 96.536) (end 107.076 98.78402) (width 0.25) (layer "B.Cu") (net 28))
 (segment (start 103.605 102.891416) (end 107.947208 98.549208) (width 0.25) (layer "B.Cu") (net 30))
 (segment (start 108.734 98.53) (end 107.966416 98.53) (width 0.23) (layer "B.Cu") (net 30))
 (segment (start 109.076 98.188) (end 108.734 98.53) (width 0.25) (layer "B.Cu") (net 30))
 (segment (start 109.076 96.536) (end 109.076 98.188) (width 0.25) (layer "B.Cu") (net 30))
 (segment (start 107.966416 98.53) (end 107.947208 98.549208) (width 0.23) (layer "B.Cu") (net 30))
 (segment (start 103.605 105.918) (end 103.605 102.891416) (width 0.25) (layer "B.Cu") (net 30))
 (segment (start 110.076 95.536) (end 109.076 96.536) (width 0.25) (layer "B.Cu") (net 30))
 (segment (start 111.076 97.950214) (end 111.076 96.536) (width 0.25) (layer "B.Cu") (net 32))
 (segment (start 108.152812 98.98) (end 110.046214 98.98) (width 0.25) (layer "B.Cu") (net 32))
 (segment (start 110.046214 98.98) (end 111.076 97.950214) (width 0.25) (layer "B.Cu") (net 32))
 (segment (start 104.405 105.918) (end 104.405 102.727812) (width 0.25) (layer "B.Cu") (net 32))
 (segment (start 104.405 102.727812) (end 108.152812 98.98) (width 0.25) (layer "B.Cu") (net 32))
 (segment (start 111.076 96.536) (end 112.076 95.536) (width 0.25) (layer "B.Cu") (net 32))
 (segment (start 111.596214 99.43) (end 113.076 97.950214) (width 0.25) (layer "B.Cu") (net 34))
 (segment (start 113.076 96.536) (end 114.076 95.536) (width 0.25) (layer "B.Cu") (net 34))
 (segment (start 113.076 97.950214) (end 113.076 96.536) (width 0.25) (layer "B.Cu") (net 34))
 (segment (start 108.339208 99.43) (end 111.596214 99.43) (width 0.25) (layer "B.Cu") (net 34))
 (segment (start 105.205 105.918) (end 105.205 102.564208) (width 0.25) (layer "B.Cu") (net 34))
 (segment (start 105.205 102.564208) (end 108.339208 99.43) (width 0.25) (layer "B.Cu") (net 34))
 (segment (start 115.076 96.536) (end 116.076 95.536) (width 0.25) (layer "B.Cu") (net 36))
 (segment (start 115.076 97.950214) (end 115.076 96.536) (width 0.25) (layer "B.Cu") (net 36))
 (segment (start 113.146214 99.88) (end 115.076 97.950214) (width 0.25) (layer "B.Cu") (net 36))
 (segment (start 106.005 102.400604) (end 108.525604 99.88) (width 0.25) (layer "B.Cu") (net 36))
 (segment (start 106.005 105.918) (end 106.005 102.400604) (width 0.25) (layer "B.Cu") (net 36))
 (segment (start 108.525604 99.88) (end 113.146214 99.88) (width 0.25) (layer "B.Cu") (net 36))
 (segment (start 117.076 97.950214) (end 117.076 96.536) (width 0.25) (layer "B.Cu") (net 38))
 (segment (start 114.696214 100.33) (end 117.076 97.950214) (width 0.25) (layer "B.Cu") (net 38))
 (segment (start 117.076 96.536) (end 118.076 95.536) (width 0.25) (layer "B.Cu") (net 38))
 (segment (start 108.712 100.33) (end 114.696214 100.33) (width 0.25) (layer "B.Cu") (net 38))
 (segment (start 106.805 105.918) (end 106.805 102.237) (width 0.25) (layer "B.Cu") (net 38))
 (segment (start 106.805 102.237) (end 108.712 100.33) (width 0.25) (layer "B.Cu") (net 38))
 (segment (start 107.605 105.918) (end 106.805 105.918) (width 0.25) (layer "B.Cu") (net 38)))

